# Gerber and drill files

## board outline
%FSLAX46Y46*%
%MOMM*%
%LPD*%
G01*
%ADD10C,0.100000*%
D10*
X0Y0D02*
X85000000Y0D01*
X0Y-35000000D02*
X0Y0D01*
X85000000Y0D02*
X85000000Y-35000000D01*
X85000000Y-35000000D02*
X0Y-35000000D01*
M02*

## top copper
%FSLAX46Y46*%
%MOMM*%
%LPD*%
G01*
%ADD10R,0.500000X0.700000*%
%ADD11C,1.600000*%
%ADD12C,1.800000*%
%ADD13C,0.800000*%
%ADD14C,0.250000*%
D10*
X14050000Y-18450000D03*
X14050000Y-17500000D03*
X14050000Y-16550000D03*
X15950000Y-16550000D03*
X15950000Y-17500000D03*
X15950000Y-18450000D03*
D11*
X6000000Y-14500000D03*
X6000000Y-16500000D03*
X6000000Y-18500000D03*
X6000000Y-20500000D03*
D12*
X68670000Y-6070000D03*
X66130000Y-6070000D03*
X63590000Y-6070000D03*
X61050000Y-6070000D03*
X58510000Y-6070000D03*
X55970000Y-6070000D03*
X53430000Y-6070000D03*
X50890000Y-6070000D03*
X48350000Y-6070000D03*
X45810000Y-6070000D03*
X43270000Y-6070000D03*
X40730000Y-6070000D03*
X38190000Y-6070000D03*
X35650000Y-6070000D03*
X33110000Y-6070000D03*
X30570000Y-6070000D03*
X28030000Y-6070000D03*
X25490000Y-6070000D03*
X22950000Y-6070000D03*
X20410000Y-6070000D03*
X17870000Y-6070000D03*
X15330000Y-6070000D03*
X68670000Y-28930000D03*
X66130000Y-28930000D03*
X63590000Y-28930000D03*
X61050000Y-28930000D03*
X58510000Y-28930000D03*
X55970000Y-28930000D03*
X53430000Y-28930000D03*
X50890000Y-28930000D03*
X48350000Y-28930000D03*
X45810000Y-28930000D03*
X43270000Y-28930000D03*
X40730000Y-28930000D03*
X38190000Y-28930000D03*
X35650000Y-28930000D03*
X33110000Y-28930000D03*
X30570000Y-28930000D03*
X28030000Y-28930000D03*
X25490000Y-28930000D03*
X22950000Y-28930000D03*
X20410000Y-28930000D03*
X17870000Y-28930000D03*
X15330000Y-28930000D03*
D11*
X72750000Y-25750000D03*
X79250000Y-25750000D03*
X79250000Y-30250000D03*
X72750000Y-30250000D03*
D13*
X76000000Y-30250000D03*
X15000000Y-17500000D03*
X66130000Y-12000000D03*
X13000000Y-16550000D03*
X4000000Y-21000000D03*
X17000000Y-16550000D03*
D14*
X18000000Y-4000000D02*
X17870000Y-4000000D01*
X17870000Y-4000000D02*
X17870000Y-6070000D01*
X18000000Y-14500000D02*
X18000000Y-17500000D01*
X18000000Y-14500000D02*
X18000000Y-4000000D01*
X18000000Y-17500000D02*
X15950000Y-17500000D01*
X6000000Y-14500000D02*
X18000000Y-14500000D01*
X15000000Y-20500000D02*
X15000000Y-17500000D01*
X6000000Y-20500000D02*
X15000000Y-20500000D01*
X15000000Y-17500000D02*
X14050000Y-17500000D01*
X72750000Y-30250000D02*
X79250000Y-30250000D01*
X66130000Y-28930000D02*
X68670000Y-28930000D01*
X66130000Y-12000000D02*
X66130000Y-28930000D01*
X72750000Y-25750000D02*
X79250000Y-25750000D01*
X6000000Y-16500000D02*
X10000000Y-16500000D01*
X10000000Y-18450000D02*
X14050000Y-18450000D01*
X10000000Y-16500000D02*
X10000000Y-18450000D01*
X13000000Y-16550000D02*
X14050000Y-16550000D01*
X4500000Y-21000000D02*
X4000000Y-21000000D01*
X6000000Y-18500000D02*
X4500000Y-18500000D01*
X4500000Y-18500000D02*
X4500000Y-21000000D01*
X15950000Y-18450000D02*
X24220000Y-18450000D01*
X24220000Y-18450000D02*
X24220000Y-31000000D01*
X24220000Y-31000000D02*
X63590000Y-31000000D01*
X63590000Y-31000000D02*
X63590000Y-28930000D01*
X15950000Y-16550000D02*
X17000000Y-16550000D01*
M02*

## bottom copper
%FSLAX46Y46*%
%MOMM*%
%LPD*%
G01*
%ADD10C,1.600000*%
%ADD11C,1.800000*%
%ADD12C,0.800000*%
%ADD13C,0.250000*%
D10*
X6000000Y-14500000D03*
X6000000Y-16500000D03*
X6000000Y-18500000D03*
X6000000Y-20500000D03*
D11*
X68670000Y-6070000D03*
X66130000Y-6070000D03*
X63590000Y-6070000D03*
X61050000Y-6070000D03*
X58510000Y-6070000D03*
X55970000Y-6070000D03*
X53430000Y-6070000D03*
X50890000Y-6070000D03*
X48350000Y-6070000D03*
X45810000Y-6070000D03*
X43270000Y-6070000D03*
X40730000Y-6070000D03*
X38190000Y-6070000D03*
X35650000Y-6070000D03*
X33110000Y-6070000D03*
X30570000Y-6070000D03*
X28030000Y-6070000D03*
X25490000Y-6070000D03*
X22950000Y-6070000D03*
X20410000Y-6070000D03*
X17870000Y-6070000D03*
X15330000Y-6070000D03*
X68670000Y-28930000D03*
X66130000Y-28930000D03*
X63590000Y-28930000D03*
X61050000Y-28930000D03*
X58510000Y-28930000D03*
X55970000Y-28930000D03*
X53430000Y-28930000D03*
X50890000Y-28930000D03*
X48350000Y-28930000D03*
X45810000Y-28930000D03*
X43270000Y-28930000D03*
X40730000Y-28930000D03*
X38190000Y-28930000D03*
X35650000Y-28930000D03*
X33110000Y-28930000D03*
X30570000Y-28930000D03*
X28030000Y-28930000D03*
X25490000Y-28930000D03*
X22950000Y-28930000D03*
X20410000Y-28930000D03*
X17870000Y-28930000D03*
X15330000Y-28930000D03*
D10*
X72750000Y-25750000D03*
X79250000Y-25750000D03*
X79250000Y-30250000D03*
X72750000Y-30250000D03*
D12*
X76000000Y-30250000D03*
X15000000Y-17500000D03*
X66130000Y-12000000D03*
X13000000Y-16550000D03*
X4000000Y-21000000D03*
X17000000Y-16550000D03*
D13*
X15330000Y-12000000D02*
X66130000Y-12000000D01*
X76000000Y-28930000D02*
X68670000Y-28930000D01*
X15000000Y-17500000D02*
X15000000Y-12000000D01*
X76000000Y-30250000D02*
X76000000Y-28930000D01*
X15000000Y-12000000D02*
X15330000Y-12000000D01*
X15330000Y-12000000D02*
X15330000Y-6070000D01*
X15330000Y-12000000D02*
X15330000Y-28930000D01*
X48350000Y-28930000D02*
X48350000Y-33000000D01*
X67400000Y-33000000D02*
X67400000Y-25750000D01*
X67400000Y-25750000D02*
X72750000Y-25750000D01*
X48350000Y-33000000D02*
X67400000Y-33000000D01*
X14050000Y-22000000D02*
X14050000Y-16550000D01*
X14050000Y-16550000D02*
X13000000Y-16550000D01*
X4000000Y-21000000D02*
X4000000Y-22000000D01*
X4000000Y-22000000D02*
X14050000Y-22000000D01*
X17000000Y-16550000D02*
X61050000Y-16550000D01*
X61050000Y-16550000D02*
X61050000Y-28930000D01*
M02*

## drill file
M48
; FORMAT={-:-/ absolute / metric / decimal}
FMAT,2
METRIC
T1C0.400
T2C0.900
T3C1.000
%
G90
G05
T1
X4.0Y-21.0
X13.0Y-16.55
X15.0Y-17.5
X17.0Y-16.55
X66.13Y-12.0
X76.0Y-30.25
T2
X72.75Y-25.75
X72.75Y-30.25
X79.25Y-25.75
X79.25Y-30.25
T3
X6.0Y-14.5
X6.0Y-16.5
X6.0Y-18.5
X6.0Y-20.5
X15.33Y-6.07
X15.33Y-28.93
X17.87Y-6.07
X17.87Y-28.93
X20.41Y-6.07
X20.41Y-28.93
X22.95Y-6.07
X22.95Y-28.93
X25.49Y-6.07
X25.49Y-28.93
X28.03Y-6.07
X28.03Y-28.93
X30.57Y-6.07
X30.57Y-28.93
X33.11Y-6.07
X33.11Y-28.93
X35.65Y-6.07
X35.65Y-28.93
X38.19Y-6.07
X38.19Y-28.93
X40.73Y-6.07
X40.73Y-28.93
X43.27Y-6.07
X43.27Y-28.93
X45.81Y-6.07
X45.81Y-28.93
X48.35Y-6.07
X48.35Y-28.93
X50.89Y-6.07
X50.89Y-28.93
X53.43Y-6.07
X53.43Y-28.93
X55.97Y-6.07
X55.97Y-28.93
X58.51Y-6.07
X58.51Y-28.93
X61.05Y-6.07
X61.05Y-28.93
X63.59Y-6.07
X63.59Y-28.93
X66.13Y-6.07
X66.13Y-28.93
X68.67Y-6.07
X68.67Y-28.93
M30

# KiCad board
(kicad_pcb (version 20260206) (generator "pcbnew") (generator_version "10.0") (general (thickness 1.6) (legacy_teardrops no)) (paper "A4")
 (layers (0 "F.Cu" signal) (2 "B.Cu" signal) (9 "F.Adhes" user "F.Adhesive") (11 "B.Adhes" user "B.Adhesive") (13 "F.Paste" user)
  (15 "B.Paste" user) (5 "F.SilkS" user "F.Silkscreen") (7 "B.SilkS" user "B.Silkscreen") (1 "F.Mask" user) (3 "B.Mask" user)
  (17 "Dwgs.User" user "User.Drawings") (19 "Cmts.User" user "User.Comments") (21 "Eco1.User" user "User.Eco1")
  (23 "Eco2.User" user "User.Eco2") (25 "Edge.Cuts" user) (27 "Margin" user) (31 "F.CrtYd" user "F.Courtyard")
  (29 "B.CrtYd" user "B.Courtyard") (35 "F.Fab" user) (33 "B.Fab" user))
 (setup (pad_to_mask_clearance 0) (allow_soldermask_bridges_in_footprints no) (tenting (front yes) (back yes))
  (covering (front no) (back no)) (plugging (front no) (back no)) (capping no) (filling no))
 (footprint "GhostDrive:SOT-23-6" (layer "F.Cu") (at 15 17.5)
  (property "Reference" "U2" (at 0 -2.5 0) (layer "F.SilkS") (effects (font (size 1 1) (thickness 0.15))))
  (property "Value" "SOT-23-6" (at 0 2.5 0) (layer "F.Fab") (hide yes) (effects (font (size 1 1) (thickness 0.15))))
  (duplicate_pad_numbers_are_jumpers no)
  (pad "1" smd rect (at -0.95 0.95) (size 0.5 0.7) (layers "F.Cu" "F.Mask" "F.Paste") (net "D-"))
  (pad "2" smd rect (at -0.95 0) (size 0.5 0.7) (layers "F.Cu" "F.Mask" "F.Paste") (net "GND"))
  (pad "3" smd rect (at -0.95 -0.95) (size 0.5 0.7) (layers "F.Cu" "F.Mask" "F.Paste") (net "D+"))
  (pad "4" smd rect (at 0.95 -0.95) (size 0.5 0.7) (layers "F.Cu" "F.Mask" "F.Paste") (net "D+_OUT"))
  (pad "5" smd rect (at 0.95 0) (size 0.5 0.7) (layers "F.Cu" "F.Mask" "F.Paste") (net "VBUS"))
  (pad "6" smd rect (at 0.95 0.95) (size 0.5 0.7) (layers "F.Cu" "F.Mask" "F.Paste") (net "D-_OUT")))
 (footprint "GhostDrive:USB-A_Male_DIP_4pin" (layer "F.Cu") (at 6 17.5)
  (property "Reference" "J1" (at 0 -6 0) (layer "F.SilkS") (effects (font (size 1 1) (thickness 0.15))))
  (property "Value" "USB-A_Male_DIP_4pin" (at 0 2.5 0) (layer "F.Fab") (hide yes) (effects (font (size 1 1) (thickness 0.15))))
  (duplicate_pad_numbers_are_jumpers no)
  (pad "1" thru_hole circle (at 0 -3) (size 1.6 1.6) (drill 1) (layers "*.Cu" "*.Mask") (remove_unused_layers no) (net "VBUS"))
  (pad "2" thru_hole circle (at 0 -1) (size 1.6 1.6) (drill 1) (layers "*.Cu" "*.Mask") (remove_unused_layers no) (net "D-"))
  (pad "3" thru_hole circle (at 0 1) (size 1.6 1.6) (drill 1) (layers "*.Cu" "*.Mask") (remove_unused_layers no) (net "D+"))
  (pad "4" thru_hole circle (at 0 3) (size 1.6 1.6) (drill 1) (layers "*.Cu" "*.Mask") (remove_unused_layers no) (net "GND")))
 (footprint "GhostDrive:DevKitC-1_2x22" (layer "F.Cu") (at 42 17.5)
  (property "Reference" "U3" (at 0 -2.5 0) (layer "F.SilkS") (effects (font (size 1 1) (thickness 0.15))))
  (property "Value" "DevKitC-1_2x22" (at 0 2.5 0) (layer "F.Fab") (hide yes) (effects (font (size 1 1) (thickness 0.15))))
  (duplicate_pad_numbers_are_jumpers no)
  (pad "1" thru_hole circle (at 26.67 -11.43) (size 1.8 1.8) (drill 1) (layers "*.Cu" "*.Mask") (remove_unused_layers no))
  (pad "2" thru_hole circle (at 24.13 -11.43) (size 1.8 1.8) (drill 1) (layers "*.Cu" "*.Mask") (remove_unused_layers no))
  (pad "3" thru_hole circle (at 21.59 -11.43) (size 1.8 1.8) (drill 1) (layers "*.Cu" "*.Mask") (remove_unused_layers no))
  (pad "4" thru_hole circle (at 19.05 -11.43) (size 1.8 1.8) (drill 1) (layers "*.Cu" "*.Mask") (remove_unused_layers no))
  (pad "5" thru_hole circle (at 16.51 -11.43) (size 1.8 1.8) (drill 1) (layers "*.Cu" "*.Mask") (remove_unused_layers no))
  (pad "6" thru_hole circle (at 13.97 -11.43) (size 1.8 1.8) (drill 1) (layers "*.Cu" "*.Mask") (remove_unused_layers no))
  (pad "7" thru_hole circle (at 11.43 -11.43) (size 1.8 1.8) (drill 1) (layers "*.Cu" "*.Mask") (remove_unused_layers no))
  (pad "8" thru_hole circle (at 8.89 -11.43) (size 1.8 1.8) (drill 1) (layers "*.Cu" "*.Mask") (remove_unused_layers no))
  (pad "9" thru_hole circle (at 6.35 -11.43) (size 1.8 1.8) (drill 1) (layers "*.Cu" "*.Mask") (remove_unused_layers no))
  (pad "10" thru_hole circle (at 3.81 -11.43) (size 1.8 1.8) (drill 1) (layers "*.Cu" "*.Mask") (remove_unused_layers no))
  (pad "11" thru_hole circle (at 1.27 -11.43) (size 1.8 1.8) (drill 1) (layers "*.Cu" "*.Mask") (remove_unused_layers no))
  (pad "12" thru_hole circle (at -1.27 -11.43) (size 1.8 1.8) (drill 1) (layers "*.Cu" "*.Mask") (remove_unused_layers no))
  (pad "13" thru_hole circle (at -3.81 -11.43) (size 1.8 1.8) (drill 1) (layers "*.Cu" "*.Mask") (remove_unused_layers no))
  (pad "14" thru_hole circle (at -6.35 -11.43) (size 1.8 1.8) (drill 1) (layers "*.Cu" "*.Mask") (remove_unused_layers no))
  (pad "15" thru_hole circle (at -8.89 -11.43) (size 1.8 1.8) (drill 1) (layers "*.Cu" "*.Mask") (remove_unused_layers no))
  (pad "16" thru_hole circle (at -11.43 -11.43) (size 1.8 1.8) (drill 1) (layers "*.Cu" "*.Mask") (remove_unused_layers no))
  (pad "17" thru_hole circle (at -13.97 -11.43) (size 1.8 1.8) (drill 1) (layers "*.Cu" "*.Mask") (remove_unused_layers no))
  (pad "18" thru_hole circle (at -16.51 -11.43) (size 1.8 1.8) (drill 1) (layers "*.Cu" "*.Mask") (remove_unused_layers no))
  (pad "19" thru_hole circle (at -19.05 -11.43) (size 1.8 1.8) (drill 1) (layers "*.Cu" "*.Mask") (remove_unused_layers no))
  (pad "20" thru_hole circle (at -21.59 -11.43) (size 1.8 1.8) (drill 1) (layers "*.Cu" "*.Mask") (remove_unused_layers no))
  (pad "21" thru_hole circle (at -24.13 -11.43) (size 1.8 1.8) (drill 1) (layers "*.Cu" "*.Mask") (remove_unused_layers no) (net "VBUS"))
  (pad "22" thru_hole circle (at -26.67 -11.43) (size 1.8 1.8) (drill 1) (layers "*.Cu" "*.Mask") (remove_unused_layers no) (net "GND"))
  (pad "23" thru_hole circle (at 26.67 11.43) (size 1.8 1.8) (drill 1) (layers "*.Cu" "*.Mask") (remove_unused_layers no) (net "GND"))
  (pad "24" thru_hole circle (at 24.13 11.43) (size 1.8 1.8) (drill 1) (layers "*.Cu" "*.Mask") (remove_unused_layers no) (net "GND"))
  (pad "25" thru_hole circle (at 21.59 11.43) (size 1.8 1.8) (drill 1) (layers "*.Cu" "*.Mask") (remove_unused_layers no) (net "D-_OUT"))
  (pad "26" thru_hole circle (at 19.05 11.43) (size 1.8 1.8) (drill 1) (layers "*.Cu" "*.Mask") (remove_unused_layers no) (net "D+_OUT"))
  (pad "27" thru_hole circle (at 16.51 11.43) (size 1.8 1.8) (drill 1) (layers "*.Cu" "*.Mask") (remove_unused_layers no))
  (pad "28" thru_hole circle (at 13.97 11.43) (size 1.8 1.8) (drill 1) (layers "*.Cu" "*.Mask") (remove_unused_layers no))
  (pad "29" thru_hole circle (at 11.43 11.43) (size 1.8 1.8) (drill 1) (layers "*.Cu" "*.Mask") (remove_unused_layers no))
  (pad "30" thru_hole circle (at 8.89 11.43) (size 1.8 1.8) (drill 1) (layers "*.Cu" "*.Mask") (remove_unused_layers no))
  (pad "31" thru_hole circle (at 6.35 11.43) (size 1.8 1.8) (drill 1) (layers "*.Cu" "*.Mask") (remove_unused_layers no) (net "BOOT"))
  (pad "32" thru_hole circle (at 3.81 11.43) (size 1.8 1.8) (drill 1) (layers "*.Cu" "*.Mask") (remove_unused_layers no))
  (pad "33" thru_hole circle (at 1.27 11.43) (size 1.8 1.8) (drill 1) (layers "*.Cu" "*.Mask") (remove_unused_layers no))
  (pad "34" thru_hole circle (at -1.27 11.43) (size 1.8 1.8) (drill 1) (layers "*.Cu" "*.Mask") (remove_unused_layers no))
  (pad "35" thru_hole circle (at -3.81 11.43) (size 1.8 1.8) (drill 1) (layers "*.Cu" "*.Mask") (remove_unused_layers no))
  (pad "36" thru_hole circle (at -6.35 11.43) (size 1.8 1.8) (drill 1) (layers "*.Cu" "*.Mask") (remove_unused_layers no))
  (pad "37" thru_hole circle (at -8.89 11.43) (size 1.8 1.8) (drill 1) (layers "*.Cu" "*.Mask") (remove_unused_layers no))
  (pad "38" thru_hole circle (at -11.43 11.43) (size 1.8 1.8) (drill 1) (layers "*.Cu" "*.Mask") (remove_unused_layers no))
  (pad "39" thru_hole circle (at -13.97 11.43) (size 1.8 1.8) (drill 1) (layers "*.Cu" "*.Mask") (remove_unused_layers no))
  (pad "40" thru_hole circle (at -16.51 11.43) (size 1.8 1.8) (drill 1) (layers "*.Cu" "*.Mask") (remove_unused_layers no))
  (pad "41" thru_hole circle (at -19.05 11.43) (size 1.8 1.8) (drill 1) (layers "*.Cu" "*.Mask") (remove_unused_layers no))
  (pad "42" thru_hole circle (at -21.59 11.43) (size 1.8 1.8) (drill 1) (layers "*.Cu" "*.Mask") (remove_unused_layers no))
  (pad "43" thru_hole circle (at -24.13 11.43) (size 1.8 1.8) (drill 1) (layers "*.Cu" "*.Mask") (remove_unused_layers no))
  (pad "44" thru_hole circle (at -26.67 11.43) (size 1.8 1.8) (drill 1) (layers "*.Cu" "*.Mask") (remove_unused_layers no) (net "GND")))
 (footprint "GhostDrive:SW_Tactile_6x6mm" (layer "F.Cu") (at 76 28)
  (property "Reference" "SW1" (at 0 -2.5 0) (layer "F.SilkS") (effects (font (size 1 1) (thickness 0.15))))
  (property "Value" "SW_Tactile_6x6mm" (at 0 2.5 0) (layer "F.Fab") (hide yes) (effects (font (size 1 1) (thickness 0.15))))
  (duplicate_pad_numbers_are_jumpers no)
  (pad "1" thru_hole circle (at -3.25 -2.25) (size 1.6 1.6) (drill 0.9) (layers "*.Cu" "*.Mask") (remove_unused_layers no) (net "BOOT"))
  (pad "2" thru_hole circle (at 3.25 -2.25) (size 1.6 1.6) (drill 0.9) (layers "*.Cu" "*.Mask") (remove_unused_layers no) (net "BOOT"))
  (pad "3" thru_hole circle (at 3.25 2.25) (size 1.6 1.6) (drill 0.9) (layers "*.Cu" "*.Mask") (remove_unused_layers no) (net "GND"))
  (pad "4" thru_hole circle (at -3.25 2.25) (size 1.6 1.6) (drill 0.9) (layers "*.Cu" "*.Mask") (remove_unused_layers no) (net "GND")))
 (gr_line (start 0 0) (end 85 0) (stroke (width 0.1) (type solid)) (layer "Edge.Cuts"))
 (gr_line (start 0 35) (end 0 0) (stroke (width 0.1) (type solid)) (layer "Edge.Cuts"))
 (gr_line (start 85 0) (end 85 35) (stroke (width 0.1) (type solid)) (layer "Edge.Cuts"))
 (gr_line (start 85 35) (end 0 35) (stroke (width 0.1) (type solid)) (layer "Edge.Cuts"))
 (segment (start 18 4) (end 17.87 4) (width 0.25) (layer "F.Cu") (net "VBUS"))
 (segment (start 17.87 4) (end 17.87 6.07) (width 0.25) (layer "F.Cu") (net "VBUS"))
 (segment (start 18 14.5) (end 18 17.5) (width 0.25) (layer "F.Cu") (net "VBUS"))
 (segment (start 18 14.5) (end 18 4) (width 0.25) (layer "F.Cu") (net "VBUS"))
 (segment (start 18 17.5) (end 15.95 17.5) (width 0.25) (layer "F.Cu") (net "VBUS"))
 (segment (start 6 14.5) (end 18 14.5) (width 0.25) (layer "F.Cu") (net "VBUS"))
 (segment (start 15 20.5) (end 15 17.5) (width 0.25) (layer "F.Cu") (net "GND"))
 (segment (start 6 20.5) (end 15 20.5) (width 0.25) (layer "F.Cu") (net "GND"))
 (segment (start 15 17.5) (end 14.05 17.5) (width 0.25) (layer "F.Cu") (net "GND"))
 (segment (start 72.75 30.25) (end 79.25 30.25) (width 0.25) (layer "F.Cu") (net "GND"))
 (segment (start 66.13 28.93) (end 68.67 28.93) (width 0.25) (layer "F.Cu") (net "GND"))
 (segment (start 66.13 12) (end 66.13 28.93) (width 0.25) (layer "F.Cu") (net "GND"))
 (via (at 76 30.25) (size 0.8) (drill 0.4) (layers "F.Cu" "B.Cu") (capping no) (covering (front no) (back no))
  (plugging (front no) (back no)) (filling no) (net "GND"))
 (via (at 15 17.5) (size 0.8) (drill 0.4) (layers "F.Cu" "B.Cu") (capping no) (covering (front no) (back no))
  (plugging (front no) (back no)) (filling no) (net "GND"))
 (via (at 66.13 12) (size 0.8) (drill 0.4) (layers "F.Cu" "B.Cu") (capping no) (covering (front no) (back no))
  (plugging (front no) (back no)) (filling no) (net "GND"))
 (segment (start 15.33 12) (end 66.13 12) (width 0.25) (layer "B.Cu") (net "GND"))
 (segment (start 76 28.93) (end 68.67 28.93) (width 0.25) (layer "B.Cu") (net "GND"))
 (segment (start 15 17.5) (end 15 12) (width 0.25) (layer "B.Cu") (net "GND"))
 (segment (start 76 30.25) (end 76 28.93) (width 0.25) (layer "B.Cu") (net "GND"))
 (segment (start 15 12) (end 15.33 12) (width 0.25) (layer "B.Cu") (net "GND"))
 (segment (start 15.33 12) (end 15.33 6.07) (width 0.25) (layer "B.Cu") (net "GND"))
 (segment (start 15.33 12) (end 15.33 28.93) (width 0.25) (layer "B.Cu") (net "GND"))
 (segment (start 72.75 25.75) (end 79.25 25.75) (width 0.25) (layer "F.Cu") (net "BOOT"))
 (segment (start 48.35 28.93) (end 48.35 33) (width 0.25) (layer "B.Cu") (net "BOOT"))
 (segment (start 67.4 33) (end 67.4 25.75) (width 0.25) (layer "B.Cu") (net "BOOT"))
 (segment (start 67.4 25.75) (end 72.75 25.75) (width 0.25) (layer "B.Cu") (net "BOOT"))
 (segment (start 48.35 33) (end 67.4 33) (width 0.25) (layer "B.Cu") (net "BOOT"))
 (segment (start 6 16.5) (end 10 16.5) (width 0.25) (layer "F.Cu") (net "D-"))
 (segment (start 10 18.45) (end 14.05 18.45) (width 0.25) (layer "F.Cu") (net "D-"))
 (segment (start 10 16.5) (end 10 18.45) (width 0.25) (layer "F.Cu") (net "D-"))
 (segment (start 13 16.55) (end 14.05 16.55) (width 0.25) (layer "F.Cu") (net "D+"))
 (segment (start 4.5 21) (end 4 21) (width 0.25) (layer "F.Cu") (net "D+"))
 (segment (start 6 18.5) (end 4.5 18.5) (width 0.25) (layer "F.Cu") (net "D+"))
 (segment (start 4.5 18.5) (end 4.5 21) (width 0.25) (layer "F.Cu") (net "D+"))
 (via (at 13 16.55) (size 0.8) (drill 0.4) (layers "F.Cu" "B.Cu") (capping no) (covering (front no) (back no))
  (plugging (front no) (back no)) (filling no) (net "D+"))
 (via (at 4 21) (size 0.8) (drill 0.4) (layers "F.Cu" "B.Cu") (capping no) (covering (front no) (back no)) (plugging (front no) (back no))
  (filling no) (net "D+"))
 (segment (start 14.05 22) (end 14.05 16.55) (width 0.25) (layer "B.Cu") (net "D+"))
 (segment (start 14.05 16.55) (end 13 16.55) (width 0.25) (layer "B.Cu") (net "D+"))
 (segment (start 4 21) (end 4 22) (width 0.25) (layer "B.Cu") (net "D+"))
 (segment (start 4 22) (end 14.05 22) (width 0.25) (layer "B.Cu") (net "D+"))
 (segment (start 15.95 18.45) (end 24.22 18.45) (width 0.25) (layer "F.Cu") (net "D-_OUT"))
 (segment (start 24.22 18.45) (end 24.22 31) (width 0.25) (layer "F.Cu") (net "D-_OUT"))
 (segment (start 24.22 31) (end 63.59 31) (width 0.25) (layer "F.Cu") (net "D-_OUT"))
 (segment (start 63.59 31) (end 63.59 28.93) (width 0.25) (layer "F.Cu") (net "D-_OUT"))
 (segment (start 15.95 16.55) (end 17 16.55) (width 0.25) (layer "F.Cu") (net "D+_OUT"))
 (via (at 17 16.55) (size 0.8) (drill 0.4) (layers "F.Cu" "B.Cu") (capping no) (covering (front no) (back no))
  (plugging (front no) (back no)) (filling no) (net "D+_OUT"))
 (segment (start 17 16.55) (end 61.05 16.55) (width 0.25) (layer "B.Cu") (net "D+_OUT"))
 (segment (start 61.05 16.55) (end 61.05 28.93) (width 0.25) (layer "B.Cu") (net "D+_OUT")))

